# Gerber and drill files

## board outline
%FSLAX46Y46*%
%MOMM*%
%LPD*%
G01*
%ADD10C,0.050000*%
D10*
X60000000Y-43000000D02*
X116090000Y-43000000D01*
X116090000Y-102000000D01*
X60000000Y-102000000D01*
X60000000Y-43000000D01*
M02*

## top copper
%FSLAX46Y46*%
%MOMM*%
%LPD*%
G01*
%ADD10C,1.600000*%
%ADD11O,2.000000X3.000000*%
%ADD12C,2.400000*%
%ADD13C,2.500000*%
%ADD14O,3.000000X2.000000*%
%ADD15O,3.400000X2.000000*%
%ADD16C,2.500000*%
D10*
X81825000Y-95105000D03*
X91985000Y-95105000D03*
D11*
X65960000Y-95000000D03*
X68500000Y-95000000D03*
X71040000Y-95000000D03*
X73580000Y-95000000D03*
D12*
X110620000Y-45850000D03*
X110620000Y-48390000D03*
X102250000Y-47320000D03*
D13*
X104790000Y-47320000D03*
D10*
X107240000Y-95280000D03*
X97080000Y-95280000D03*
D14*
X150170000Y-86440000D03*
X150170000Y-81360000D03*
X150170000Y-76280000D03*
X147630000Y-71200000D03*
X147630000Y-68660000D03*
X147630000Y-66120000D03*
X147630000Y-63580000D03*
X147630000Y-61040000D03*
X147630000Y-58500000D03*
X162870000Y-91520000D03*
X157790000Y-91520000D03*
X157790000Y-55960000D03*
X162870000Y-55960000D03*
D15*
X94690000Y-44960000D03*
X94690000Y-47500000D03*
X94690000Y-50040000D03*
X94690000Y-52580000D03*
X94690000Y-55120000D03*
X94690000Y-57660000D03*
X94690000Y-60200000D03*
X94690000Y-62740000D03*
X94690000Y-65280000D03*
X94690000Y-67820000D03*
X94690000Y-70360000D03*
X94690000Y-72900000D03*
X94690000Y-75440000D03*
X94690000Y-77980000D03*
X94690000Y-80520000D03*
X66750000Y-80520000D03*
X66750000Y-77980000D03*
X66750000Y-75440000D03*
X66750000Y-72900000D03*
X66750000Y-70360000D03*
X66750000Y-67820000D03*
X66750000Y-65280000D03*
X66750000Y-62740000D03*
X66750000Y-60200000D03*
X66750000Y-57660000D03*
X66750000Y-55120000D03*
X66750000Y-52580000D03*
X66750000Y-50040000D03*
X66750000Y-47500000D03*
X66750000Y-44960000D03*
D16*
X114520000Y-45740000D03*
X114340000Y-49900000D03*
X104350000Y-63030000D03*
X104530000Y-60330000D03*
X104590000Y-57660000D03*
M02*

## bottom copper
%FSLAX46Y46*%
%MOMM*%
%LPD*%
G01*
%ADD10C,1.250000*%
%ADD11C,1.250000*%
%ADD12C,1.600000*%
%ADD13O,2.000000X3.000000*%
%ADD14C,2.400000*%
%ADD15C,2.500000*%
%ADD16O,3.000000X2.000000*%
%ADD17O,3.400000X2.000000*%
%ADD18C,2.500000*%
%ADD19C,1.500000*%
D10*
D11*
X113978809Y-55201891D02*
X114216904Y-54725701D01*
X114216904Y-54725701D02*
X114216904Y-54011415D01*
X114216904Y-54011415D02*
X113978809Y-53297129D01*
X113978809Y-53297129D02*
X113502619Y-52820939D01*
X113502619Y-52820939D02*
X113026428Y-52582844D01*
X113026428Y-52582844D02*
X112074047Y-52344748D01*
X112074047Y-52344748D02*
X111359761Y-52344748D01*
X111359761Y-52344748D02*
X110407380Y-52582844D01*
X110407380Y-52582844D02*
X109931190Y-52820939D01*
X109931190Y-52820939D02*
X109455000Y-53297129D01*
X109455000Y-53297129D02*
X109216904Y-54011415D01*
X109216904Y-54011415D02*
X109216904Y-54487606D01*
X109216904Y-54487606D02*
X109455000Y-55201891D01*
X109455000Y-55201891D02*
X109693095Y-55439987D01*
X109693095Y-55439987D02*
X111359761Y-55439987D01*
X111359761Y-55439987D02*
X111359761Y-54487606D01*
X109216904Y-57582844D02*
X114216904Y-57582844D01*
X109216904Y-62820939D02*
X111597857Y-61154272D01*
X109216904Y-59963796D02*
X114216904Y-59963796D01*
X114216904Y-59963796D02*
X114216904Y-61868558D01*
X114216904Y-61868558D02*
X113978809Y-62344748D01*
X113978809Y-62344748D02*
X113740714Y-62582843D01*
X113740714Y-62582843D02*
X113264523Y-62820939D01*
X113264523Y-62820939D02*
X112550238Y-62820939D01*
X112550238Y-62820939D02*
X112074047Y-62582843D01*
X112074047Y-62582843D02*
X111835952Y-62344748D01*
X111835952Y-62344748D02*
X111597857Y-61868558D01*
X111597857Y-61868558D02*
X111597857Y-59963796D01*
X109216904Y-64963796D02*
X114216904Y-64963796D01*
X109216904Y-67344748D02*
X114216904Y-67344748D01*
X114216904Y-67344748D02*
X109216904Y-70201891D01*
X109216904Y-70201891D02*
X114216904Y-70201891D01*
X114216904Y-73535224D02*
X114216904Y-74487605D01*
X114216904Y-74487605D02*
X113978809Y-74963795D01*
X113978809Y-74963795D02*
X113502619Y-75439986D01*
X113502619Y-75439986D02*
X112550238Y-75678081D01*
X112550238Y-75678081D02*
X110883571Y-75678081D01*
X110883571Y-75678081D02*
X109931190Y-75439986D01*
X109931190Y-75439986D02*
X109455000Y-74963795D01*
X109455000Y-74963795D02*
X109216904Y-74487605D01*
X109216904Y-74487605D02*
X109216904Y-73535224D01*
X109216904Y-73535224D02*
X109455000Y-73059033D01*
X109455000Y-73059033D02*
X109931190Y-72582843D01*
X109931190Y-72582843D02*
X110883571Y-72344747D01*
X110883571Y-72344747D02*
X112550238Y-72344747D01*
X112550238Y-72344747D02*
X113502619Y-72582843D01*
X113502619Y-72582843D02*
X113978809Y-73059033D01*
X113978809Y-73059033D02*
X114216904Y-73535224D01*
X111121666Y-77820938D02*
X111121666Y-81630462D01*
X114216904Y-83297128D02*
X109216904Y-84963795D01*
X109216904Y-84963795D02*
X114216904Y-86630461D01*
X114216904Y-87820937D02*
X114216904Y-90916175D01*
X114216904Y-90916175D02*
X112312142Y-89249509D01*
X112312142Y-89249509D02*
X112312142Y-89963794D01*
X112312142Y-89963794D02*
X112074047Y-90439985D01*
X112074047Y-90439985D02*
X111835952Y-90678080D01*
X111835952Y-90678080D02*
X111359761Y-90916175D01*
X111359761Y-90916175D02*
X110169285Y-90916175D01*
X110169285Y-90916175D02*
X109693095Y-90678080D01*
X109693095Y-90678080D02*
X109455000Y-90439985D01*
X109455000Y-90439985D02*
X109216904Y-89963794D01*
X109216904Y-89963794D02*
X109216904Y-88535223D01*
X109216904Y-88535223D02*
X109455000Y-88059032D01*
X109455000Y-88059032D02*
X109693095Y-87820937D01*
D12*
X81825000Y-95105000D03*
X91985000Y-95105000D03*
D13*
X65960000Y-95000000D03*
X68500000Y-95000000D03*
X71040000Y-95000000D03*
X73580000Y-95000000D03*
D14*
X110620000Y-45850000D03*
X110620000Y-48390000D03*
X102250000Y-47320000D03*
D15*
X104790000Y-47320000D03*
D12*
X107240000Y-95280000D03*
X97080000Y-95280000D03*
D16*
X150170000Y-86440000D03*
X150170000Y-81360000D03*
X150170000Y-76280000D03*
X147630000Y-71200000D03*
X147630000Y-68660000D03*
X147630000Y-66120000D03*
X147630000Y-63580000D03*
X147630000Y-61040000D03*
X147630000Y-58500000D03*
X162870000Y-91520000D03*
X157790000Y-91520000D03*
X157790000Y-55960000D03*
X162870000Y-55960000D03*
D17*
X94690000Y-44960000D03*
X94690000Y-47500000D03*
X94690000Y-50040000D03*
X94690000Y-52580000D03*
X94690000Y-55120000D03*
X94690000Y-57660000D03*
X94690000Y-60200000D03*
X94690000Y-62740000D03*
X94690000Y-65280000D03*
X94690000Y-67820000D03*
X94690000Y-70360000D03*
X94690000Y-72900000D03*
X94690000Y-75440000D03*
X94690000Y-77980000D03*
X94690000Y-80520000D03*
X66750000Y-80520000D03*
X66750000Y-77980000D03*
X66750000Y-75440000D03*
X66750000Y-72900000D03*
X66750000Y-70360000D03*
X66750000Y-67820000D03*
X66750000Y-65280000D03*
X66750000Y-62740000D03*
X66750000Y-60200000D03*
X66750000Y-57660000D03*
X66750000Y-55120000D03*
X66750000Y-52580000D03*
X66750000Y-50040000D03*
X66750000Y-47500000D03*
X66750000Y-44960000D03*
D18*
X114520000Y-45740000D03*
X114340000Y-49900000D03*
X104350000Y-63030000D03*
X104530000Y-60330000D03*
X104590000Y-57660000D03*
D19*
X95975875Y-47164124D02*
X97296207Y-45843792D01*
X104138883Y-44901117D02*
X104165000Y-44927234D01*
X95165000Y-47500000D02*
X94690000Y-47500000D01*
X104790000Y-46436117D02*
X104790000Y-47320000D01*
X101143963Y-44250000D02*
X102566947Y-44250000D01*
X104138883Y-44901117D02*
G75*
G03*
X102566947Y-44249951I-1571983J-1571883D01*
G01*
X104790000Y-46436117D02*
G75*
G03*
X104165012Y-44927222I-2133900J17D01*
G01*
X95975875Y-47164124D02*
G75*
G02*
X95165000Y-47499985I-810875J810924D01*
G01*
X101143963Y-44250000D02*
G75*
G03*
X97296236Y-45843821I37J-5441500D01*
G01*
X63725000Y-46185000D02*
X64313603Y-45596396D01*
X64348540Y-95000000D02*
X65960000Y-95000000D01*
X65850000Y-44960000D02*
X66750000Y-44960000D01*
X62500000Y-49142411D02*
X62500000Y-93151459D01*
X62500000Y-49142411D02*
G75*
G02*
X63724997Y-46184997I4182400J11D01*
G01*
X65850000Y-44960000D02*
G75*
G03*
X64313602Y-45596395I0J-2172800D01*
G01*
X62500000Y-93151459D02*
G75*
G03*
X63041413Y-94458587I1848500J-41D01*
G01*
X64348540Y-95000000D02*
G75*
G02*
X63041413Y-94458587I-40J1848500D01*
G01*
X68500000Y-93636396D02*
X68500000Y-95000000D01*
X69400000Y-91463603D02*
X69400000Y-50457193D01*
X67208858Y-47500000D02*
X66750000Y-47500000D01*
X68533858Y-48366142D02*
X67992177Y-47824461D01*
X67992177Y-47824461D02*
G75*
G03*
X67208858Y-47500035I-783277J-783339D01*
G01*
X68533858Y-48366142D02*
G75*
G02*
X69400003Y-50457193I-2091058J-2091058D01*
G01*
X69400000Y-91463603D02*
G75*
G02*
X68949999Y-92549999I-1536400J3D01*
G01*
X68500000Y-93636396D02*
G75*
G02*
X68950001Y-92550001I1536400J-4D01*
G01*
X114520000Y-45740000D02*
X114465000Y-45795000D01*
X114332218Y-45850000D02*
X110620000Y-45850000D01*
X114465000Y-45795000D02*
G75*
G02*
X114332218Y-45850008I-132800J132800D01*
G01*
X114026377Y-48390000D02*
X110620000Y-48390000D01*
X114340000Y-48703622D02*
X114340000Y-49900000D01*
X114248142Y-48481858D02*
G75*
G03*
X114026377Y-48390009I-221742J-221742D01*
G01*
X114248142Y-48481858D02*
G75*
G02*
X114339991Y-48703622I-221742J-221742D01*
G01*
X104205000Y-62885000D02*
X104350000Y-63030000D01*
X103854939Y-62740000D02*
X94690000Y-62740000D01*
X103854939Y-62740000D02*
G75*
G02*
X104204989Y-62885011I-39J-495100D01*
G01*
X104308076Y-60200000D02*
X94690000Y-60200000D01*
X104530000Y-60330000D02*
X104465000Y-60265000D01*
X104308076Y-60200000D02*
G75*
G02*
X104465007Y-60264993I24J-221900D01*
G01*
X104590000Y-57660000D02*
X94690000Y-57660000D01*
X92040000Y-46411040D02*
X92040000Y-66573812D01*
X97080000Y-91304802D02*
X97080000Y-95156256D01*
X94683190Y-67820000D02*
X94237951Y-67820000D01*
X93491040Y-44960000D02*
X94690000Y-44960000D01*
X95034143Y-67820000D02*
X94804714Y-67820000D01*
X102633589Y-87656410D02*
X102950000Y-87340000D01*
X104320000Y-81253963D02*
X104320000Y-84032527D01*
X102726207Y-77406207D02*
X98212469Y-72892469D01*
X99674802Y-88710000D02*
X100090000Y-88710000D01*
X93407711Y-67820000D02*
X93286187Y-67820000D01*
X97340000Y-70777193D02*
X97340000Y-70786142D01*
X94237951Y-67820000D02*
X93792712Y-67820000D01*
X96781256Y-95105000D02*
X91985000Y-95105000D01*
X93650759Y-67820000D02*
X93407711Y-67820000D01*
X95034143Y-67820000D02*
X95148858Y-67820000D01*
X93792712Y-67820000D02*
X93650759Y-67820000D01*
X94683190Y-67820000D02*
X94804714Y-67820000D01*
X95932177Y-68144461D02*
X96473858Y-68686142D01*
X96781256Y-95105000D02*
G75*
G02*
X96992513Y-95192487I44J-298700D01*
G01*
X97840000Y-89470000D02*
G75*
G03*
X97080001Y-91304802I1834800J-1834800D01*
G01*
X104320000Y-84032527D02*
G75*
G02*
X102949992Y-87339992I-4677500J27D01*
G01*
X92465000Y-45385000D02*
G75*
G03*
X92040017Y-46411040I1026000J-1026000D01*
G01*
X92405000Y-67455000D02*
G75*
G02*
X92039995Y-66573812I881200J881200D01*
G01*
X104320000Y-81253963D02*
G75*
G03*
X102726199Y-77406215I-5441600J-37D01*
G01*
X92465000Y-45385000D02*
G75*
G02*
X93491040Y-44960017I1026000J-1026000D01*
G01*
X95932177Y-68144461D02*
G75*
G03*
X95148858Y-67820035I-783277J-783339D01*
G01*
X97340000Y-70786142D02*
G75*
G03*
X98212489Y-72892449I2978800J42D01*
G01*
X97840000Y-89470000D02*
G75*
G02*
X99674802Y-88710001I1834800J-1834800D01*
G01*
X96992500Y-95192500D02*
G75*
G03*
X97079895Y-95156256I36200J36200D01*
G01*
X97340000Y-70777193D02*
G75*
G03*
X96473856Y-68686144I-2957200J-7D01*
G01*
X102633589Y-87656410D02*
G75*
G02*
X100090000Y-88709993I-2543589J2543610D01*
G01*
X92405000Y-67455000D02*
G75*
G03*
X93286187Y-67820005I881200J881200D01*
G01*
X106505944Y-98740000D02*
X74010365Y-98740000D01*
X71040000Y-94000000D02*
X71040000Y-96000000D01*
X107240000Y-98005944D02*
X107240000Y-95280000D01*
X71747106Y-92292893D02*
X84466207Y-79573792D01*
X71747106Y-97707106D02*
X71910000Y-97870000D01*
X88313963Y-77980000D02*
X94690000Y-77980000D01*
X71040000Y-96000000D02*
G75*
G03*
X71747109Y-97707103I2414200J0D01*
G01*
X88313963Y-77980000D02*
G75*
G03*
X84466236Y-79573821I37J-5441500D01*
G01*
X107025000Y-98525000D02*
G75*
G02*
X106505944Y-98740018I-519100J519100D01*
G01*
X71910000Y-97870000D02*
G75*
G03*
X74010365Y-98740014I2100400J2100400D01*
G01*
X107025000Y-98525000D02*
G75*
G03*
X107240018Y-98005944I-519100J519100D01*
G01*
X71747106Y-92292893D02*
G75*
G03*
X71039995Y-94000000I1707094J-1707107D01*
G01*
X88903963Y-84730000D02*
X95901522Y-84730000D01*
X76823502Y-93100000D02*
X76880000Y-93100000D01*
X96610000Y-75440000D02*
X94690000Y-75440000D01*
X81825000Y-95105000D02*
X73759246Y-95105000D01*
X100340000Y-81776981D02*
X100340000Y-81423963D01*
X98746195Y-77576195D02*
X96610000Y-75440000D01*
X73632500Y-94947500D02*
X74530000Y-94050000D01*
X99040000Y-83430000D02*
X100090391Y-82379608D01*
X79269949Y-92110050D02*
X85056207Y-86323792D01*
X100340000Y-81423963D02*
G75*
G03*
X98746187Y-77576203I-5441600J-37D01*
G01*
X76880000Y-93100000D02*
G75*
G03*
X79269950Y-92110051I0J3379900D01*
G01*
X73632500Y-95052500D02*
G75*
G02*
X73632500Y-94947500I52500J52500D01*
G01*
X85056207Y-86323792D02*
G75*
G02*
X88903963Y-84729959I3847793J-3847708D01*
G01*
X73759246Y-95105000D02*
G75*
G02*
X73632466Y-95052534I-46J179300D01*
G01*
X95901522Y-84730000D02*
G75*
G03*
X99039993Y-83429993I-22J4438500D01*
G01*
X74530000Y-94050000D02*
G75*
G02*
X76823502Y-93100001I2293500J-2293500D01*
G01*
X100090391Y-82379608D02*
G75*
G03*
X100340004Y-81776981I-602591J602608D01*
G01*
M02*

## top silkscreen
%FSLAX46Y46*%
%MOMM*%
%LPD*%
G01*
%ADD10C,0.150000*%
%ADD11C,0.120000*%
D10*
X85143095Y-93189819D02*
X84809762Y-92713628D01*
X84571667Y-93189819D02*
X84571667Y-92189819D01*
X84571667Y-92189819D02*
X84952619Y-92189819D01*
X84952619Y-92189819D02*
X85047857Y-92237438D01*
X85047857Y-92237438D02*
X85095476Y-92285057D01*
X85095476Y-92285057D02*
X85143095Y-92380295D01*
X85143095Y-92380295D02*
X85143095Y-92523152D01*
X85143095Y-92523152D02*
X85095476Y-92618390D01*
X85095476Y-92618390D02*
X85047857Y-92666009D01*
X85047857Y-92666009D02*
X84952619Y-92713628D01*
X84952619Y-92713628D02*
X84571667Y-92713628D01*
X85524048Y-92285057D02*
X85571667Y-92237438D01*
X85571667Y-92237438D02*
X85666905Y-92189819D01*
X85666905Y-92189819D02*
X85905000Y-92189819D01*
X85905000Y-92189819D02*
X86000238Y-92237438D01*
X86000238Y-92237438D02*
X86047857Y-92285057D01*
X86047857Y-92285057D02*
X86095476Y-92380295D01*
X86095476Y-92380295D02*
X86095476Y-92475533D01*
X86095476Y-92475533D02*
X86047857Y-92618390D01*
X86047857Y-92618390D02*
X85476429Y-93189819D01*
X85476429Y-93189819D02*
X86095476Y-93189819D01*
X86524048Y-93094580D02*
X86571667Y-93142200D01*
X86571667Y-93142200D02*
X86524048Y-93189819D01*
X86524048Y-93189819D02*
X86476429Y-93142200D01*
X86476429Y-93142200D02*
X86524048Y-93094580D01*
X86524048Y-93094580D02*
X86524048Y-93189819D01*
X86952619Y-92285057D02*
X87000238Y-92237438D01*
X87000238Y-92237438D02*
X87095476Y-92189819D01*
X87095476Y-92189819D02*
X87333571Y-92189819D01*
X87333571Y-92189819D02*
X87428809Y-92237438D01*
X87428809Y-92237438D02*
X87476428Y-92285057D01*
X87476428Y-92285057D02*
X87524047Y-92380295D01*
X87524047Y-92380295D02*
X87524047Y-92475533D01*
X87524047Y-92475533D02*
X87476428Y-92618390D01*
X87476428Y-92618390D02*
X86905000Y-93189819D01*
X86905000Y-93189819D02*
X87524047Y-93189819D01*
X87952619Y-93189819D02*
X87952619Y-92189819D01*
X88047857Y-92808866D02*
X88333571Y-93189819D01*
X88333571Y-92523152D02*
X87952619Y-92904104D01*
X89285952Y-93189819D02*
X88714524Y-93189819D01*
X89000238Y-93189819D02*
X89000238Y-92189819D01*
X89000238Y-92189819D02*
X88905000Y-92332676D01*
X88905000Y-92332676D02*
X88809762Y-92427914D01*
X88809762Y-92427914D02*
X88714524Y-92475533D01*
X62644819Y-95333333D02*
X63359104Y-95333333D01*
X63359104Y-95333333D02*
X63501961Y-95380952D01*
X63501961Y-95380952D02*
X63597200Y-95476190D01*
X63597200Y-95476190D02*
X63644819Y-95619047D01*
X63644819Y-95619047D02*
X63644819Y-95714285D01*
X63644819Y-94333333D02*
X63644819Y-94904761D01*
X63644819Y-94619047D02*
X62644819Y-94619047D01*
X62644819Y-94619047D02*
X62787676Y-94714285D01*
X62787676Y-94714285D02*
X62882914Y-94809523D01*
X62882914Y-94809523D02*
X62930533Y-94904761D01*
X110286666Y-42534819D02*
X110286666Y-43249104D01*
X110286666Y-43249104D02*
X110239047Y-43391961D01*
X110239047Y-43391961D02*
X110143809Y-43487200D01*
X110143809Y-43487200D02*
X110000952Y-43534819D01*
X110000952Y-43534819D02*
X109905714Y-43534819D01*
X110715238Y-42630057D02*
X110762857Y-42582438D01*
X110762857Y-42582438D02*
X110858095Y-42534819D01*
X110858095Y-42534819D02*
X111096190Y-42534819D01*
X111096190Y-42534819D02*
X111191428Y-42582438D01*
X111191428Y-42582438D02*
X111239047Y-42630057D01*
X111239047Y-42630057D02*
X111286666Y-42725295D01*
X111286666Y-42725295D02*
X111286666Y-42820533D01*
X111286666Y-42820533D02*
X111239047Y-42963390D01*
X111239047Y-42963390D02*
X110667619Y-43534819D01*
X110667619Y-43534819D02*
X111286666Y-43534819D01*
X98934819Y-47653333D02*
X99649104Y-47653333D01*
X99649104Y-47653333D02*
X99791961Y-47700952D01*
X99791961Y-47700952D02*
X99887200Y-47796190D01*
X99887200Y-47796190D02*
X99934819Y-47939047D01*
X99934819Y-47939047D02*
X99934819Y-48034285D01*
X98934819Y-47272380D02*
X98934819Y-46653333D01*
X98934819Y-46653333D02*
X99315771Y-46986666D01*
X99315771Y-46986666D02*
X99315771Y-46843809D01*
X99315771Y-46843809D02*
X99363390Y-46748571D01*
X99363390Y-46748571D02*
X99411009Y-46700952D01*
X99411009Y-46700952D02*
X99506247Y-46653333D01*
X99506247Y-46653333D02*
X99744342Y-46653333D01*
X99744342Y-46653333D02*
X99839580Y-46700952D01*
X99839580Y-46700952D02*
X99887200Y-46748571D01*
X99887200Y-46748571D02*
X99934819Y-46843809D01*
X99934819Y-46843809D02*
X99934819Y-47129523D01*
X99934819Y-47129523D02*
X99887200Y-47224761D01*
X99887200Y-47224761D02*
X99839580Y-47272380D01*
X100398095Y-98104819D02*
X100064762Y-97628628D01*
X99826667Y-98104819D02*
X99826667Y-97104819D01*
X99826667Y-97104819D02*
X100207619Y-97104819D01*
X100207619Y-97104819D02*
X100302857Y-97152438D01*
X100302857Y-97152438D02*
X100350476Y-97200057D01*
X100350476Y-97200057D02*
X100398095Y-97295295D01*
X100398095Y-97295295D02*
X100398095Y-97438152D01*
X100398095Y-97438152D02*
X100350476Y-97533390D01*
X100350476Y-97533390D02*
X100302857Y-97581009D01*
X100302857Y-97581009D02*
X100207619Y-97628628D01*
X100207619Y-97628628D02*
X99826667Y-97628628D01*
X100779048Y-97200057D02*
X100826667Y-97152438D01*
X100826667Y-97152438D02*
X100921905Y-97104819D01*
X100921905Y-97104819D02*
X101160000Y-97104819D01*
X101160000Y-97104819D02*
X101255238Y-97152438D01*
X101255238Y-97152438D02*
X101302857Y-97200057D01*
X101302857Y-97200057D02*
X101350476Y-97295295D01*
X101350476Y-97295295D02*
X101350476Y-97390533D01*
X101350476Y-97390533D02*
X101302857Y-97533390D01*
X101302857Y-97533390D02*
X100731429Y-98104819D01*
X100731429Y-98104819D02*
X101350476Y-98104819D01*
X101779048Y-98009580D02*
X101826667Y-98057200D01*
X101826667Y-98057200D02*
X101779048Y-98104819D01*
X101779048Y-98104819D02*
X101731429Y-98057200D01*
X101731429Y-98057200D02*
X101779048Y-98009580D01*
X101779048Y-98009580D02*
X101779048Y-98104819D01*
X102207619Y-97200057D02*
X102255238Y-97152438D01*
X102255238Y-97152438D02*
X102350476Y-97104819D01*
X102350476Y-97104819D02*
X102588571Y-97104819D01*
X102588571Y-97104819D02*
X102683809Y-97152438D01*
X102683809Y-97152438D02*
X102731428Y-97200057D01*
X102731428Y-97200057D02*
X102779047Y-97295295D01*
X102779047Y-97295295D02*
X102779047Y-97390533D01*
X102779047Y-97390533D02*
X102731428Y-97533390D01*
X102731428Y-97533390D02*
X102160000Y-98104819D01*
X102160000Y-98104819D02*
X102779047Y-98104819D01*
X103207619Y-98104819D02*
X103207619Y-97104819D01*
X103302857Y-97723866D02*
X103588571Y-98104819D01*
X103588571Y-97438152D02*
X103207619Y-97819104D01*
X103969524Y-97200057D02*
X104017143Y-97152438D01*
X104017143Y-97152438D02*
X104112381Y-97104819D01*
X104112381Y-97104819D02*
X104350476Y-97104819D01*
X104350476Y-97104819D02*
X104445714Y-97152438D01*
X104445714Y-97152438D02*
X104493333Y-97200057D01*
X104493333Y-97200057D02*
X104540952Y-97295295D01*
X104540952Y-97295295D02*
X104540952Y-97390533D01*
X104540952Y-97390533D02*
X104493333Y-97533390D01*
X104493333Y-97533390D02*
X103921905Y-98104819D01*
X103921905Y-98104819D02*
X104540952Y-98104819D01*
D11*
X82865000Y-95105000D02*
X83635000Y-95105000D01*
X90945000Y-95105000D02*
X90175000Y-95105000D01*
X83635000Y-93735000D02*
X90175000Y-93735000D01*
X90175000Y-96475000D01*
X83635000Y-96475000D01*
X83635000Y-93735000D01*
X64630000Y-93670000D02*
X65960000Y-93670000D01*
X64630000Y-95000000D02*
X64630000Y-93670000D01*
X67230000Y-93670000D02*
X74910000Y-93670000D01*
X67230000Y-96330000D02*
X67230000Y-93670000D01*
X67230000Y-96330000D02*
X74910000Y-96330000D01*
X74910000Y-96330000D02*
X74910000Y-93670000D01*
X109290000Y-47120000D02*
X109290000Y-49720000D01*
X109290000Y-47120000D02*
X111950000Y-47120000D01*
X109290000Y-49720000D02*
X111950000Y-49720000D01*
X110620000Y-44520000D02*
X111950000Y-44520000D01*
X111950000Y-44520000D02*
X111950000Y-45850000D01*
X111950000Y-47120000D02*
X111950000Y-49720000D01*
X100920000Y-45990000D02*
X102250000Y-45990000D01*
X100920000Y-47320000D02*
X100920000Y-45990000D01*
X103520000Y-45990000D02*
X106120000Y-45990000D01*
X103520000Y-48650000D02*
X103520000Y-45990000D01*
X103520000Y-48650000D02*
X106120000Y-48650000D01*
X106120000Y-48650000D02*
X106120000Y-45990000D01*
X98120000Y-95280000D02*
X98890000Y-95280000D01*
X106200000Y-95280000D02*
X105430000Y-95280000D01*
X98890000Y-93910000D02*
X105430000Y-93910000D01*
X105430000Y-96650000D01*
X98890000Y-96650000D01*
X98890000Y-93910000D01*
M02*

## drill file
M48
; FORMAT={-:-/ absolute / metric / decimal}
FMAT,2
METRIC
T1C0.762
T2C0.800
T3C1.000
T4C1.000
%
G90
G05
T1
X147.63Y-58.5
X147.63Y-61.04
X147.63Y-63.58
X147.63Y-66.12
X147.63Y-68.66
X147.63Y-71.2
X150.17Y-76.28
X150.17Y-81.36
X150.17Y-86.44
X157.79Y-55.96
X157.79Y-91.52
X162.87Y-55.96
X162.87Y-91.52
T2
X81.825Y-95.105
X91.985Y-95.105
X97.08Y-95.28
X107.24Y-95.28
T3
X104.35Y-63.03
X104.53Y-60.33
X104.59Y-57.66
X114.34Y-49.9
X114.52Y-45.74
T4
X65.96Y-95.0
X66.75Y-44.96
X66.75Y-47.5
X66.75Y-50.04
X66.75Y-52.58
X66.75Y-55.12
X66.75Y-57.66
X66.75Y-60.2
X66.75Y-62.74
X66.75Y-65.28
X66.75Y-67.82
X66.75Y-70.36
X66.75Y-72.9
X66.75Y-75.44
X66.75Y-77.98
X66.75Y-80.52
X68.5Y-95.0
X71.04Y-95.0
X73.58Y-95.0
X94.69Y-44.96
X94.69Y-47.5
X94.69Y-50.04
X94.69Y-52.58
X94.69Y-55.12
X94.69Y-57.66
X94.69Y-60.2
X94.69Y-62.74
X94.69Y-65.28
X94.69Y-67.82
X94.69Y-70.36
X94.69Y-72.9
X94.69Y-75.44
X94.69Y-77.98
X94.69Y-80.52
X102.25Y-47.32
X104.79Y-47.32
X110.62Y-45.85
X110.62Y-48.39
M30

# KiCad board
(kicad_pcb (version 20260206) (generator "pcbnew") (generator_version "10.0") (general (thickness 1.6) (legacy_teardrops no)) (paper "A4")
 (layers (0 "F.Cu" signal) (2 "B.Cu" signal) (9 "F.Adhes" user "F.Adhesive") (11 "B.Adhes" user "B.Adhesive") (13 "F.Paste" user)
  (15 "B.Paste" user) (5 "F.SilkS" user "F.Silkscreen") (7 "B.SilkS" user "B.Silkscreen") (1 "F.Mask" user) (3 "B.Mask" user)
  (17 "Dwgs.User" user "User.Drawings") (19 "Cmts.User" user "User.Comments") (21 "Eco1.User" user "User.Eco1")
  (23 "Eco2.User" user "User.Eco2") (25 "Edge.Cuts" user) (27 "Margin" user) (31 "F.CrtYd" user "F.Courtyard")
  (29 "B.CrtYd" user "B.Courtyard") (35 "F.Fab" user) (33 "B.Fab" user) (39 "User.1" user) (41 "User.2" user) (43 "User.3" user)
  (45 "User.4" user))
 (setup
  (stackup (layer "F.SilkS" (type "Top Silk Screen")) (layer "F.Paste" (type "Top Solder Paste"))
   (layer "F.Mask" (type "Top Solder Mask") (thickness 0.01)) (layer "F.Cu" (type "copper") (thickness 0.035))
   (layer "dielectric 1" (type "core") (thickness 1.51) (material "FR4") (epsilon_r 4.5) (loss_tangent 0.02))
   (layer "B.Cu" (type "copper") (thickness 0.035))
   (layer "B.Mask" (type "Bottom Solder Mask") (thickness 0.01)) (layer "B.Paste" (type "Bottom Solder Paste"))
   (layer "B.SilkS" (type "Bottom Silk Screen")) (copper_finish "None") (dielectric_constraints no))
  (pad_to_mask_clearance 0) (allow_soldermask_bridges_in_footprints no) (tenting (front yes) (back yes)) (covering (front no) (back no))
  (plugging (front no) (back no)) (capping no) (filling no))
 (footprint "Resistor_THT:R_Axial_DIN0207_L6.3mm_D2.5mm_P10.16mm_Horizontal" (layer "F.Cu") (at 81.825 95.105)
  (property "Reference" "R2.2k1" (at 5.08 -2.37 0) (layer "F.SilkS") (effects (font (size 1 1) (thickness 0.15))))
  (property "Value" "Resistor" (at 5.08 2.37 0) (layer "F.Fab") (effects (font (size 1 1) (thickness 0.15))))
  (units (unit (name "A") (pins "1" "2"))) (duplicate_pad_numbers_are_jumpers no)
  (fp_line (start 1.04 0) (end 1.81 0) (stroke (width 0.12) (type solid)) (layer "F.SilkS"))
  (fp_line (start 9.12 0) (end 8.35 0) (stroke (width 0.12) (type solid)) (layer "F.SilkS"))
  (fp_rect (start 1.81 -1.37) (end 8.35 1.37) (stroke (width 0.12) (type solid)) (fill no) (layer "F.SilkS"))
  (pad "1" thru_hole circle (at 0 0) (size 1.6 1.6) (drill 0.8) (layers "*.Cu" "*.Mask") (remove_unused_layers no)
   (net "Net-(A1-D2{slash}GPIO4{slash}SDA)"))
  (pad "2" thru_hole circle (at 10.16 0) (size 1.6 1.6) (drill 0.8) (layers "*.Cu" "*.Mask") (remove_unused_layers no) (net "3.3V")))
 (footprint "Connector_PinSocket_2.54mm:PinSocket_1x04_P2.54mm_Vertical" (layer "F.Cu") (at 65.96 95 90)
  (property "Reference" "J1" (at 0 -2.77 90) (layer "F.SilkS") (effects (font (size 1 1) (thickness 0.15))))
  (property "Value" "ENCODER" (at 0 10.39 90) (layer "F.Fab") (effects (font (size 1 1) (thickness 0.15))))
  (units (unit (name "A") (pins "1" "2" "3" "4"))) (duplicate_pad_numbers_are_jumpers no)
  (fp_line (start 1.33 -1.33) (end 1.33 0) (stroke (width 0.12) (type solid)) (layer "F.SilkS"))
  (fp_line (start 0 -1.33) (end 1.33 -1.33) (stroke (width 0.12) (type solid)) (layer "F.SilkS"))
  (fp_line (start 1.33 1.27) (end 1.33 8.95) (stroke (width 0.12) (type solid)) (layer "F.SilkS"))
  (fp_line (start -1.33 1.27) (end 1.33 1.27) (stroke (width 0.12) (type solid)) (layer "F.SilkS"))
  (fp_line (start -1.33 1.27) (end -1.33 8.95) (stroke (width 0.12) (type solid)) (layer "F.SilkS"))
  (fp_line (start -1.33 8.95) (end 1.33 8.95) (stroke (width 0.12) (type solid)) (layer "F.SilkS"))
  (pad "1" thru_hole oval (at 0 0 90) (size 3 2) (drill 1) (layers "*.Cu" "*.Mask") (remove_unused_layers no) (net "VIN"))
  (pad "2" thru_hole oval (at 0 2.54 90) (size 3 2) (drill 1) (layers "*.Cu" "*.Mask") (remove_unused_layers no) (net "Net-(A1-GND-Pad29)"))
  (pad "3" thru_hole oval (at 0 5.08 90) (size 3 2) (drill 1) (layers "*.Cu" "*.Mask") (remove_unused_layers no)
   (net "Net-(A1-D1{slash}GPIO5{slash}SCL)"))
  (pad "4" thru_hole oval (at 0 7.62 90) (size 3 2) (drill 1) (layers "*.Cu" "*.Mask") (remove_unused_layers no)
   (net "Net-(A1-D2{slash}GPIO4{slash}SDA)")))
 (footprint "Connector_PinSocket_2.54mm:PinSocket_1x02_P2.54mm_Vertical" (layer "F.Cu") (at 110.62 45.85)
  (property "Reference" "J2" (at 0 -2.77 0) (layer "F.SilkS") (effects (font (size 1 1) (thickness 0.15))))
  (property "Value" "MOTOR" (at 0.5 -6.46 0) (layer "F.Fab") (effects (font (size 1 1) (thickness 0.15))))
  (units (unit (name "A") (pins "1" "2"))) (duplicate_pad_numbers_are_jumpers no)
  (fp_line (start -1.33 1.27) (end -1.33 3.87) (stroke (width 0.12) (type solid)) (layer "F.SilkS"))
  (fp_line (start -1.33 1.27) (end 1.33 1.27) (stroke (width 0.12) (type solid)) (layer "F.SilkS"))
  (fp_line (start -1.33 3.87) (end 1.33 3.87) (stroke (width 0.12) (type solid)) (layer "F.SilkS"))
  (fp_line (start 0 -1.33) (end 1.33 -1.33) (stroke (width 0.12) (type solid)) (layer "F.SilkS"))
  (fp_line (start 1.33 -1.33) (end 1.33 0) (stroke (width 0.12) (type solid)) (layer "F.SilkS"))
  (fp_line (start 1.33 1.27) (end 1.33 3.87) (stroke (width 0.12) (type solid)) (layer "F.SilkS"))
  (pad "1" thru_hole circle (at 0 0) (size 2.4 2.4) (drill 1) (layers "*.Cu" "*.Mask") (remove_unused_layers no) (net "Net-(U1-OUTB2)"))
  (pad "2" thru_hole circle (at 0 2.54) (size 2.4 2.4) (drill 1) (layers "*.Cu" "*.Mask") (remove_unused_layers no) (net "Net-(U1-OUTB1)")))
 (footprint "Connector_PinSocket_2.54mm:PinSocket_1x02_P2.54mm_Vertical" (layer "F.Cu") (at 102.25 47.32 90)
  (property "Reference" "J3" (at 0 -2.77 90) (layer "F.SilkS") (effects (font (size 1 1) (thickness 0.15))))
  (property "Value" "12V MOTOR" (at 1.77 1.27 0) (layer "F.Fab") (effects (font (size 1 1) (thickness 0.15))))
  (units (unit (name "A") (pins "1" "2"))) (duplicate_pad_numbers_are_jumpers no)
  (fp_line (start 1.33 -1.33) (end 1.33 0) (stroke (width 0.12) (type solid)) (layer "F.SilkS"))
  (fp_line (start 0 -1.33) (end 1.33 -1.33) (stroke (width 0.12) (type solid)) (layer "F.SilkS"))
  (fp_line (start 1.33 1.27) (end 1.33 3.87) (stroke (width 0.12) (type solid)) (layer "F.SilkS"))
  (fp_line (start -1.33 1.27) (end 1.33 1.27) (stroke (width 0.12) (type solid)) (layer "F.SilkS"))
  (fp_line (start -1.33 1.27) (end -1.33 3.87) (stroke (width 0.12) (type solid)) (layer "F.SilkS"))
  (fp_line (start -1.33 3.87) (end 1.33 3.87) (stroke (width 0.12) (type solid)) (layer "F.SilkS"))
  (pad "1" thru_hole circle (at 0 0 90) (size 2.4 2.4) (drill 1) (layers "*.Cu" "*.Mask") (remove_unused_layers no) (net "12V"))
  (pad "2" thru_hole circle (at 0 2.54 90) (size 2.5 2.5) (drill 1) (layers "*.Cu" "*.Mask") (remove_unused_layers no) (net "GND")))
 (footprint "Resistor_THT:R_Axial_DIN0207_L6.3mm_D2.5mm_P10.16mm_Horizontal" (layer "F.Cu") (at 107.24 95.28 180)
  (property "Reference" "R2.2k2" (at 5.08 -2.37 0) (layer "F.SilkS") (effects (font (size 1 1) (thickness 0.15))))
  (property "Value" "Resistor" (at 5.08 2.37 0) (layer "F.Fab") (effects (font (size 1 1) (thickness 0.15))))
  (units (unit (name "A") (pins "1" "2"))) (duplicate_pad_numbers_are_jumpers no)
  (fp_line (start 9.12 0) (end 8.35 0) (stroke (width 0.12) (type solid)) (layer "F.SilkS"))
  (fp_line (start 1.04 0) (end 1.81 0) (stroke (width 0.12) (type solid)) (layer "F.SilkS"))
  (fp_rect (start 1.81 -1.37) (end 8.35 1.37) (stroke (width 0.12) (type solid)) (fill no) (layer "F.SilkS"))
  (pad "1" thru_hole circle (at 0 0 180) (size 1.6 1.6) (drill 0.8) (layers "*.Cu" "*.Mask") (remove_unused_layers no)
   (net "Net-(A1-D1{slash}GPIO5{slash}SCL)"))
  (pad "2" thru_hole circle (at 10.16 0 180) (size 1.6 1.6) (drill 0.8) (layers "*.Cu" "*.Mask") (remove_unused_layers no) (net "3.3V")))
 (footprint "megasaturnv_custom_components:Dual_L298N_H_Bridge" (layer "B.Cu") (at 145.09 94.06 90)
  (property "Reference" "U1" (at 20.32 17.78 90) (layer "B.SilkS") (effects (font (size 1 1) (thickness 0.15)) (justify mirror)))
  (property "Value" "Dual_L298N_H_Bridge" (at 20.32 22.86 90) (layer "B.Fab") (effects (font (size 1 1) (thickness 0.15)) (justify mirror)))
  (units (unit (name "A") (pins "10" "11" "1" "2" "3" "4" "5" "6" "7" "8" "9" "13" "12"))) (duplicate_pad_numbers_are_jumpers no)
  (pad "1" thru_hole oval (at 7.62 5.08 90) (size 2 3) (drill 0.762) (layers "*.Cu" "*.Mask") (remove_unused_layers no)
   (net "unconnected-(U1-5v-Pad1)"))
  (pad "2" thru_hole oval (at 12.7 5.08 90) (size 2 3) (drill 0.762) (layers "*.Cu" "*.Mask") (remove_unused_layers no) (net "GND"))
  (pad "3" thru_hole oval (at 17.78 5.08 90) (size 2 3) (drill 0.762) (layers "*.Cu" "*.Mask") (remove_unused_layers no) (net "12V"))
  (pad "4" thru_hole oval (at 22.86 2.54 90) (size 2 3) (drill 0.762) (layers "*.Cu" "*.Mask") (remove_unused_layers no)
   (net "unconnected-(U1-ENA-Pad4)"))
  (pad "5" thru_hole oval (at 25.4 2.54 90) (size 2 3) (drill 0.762) (layers "*.Cu" "*.Mask") (remove_unused_layers no)
   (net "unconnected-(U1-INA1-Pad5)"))
  (pad "6" thru_hole oval (at 27.94 2.54 90) (size 2 3) (drill 0.762) (layers "*.Cu" "*.Mask") (remove_unused_layers no)
   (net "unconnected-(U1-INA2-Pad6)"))
  (pad "7" thru_hole oval (at 30.48 2.54 90) (size 2 3) (drill 0.762) (layers "*.Cu" "*.Mask") (remove_unused_layers no)
   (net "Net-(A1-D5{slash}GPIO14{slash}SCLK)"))
  (pad "8" thru_hole oval (at 33.02 2.54 90) (size 2 3) (drill 0.762) (layers "*.Cu" "*.Mask") (remove_unused_layers no)
   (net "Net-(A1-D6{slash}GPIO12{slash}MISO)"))
  (pad "9" thru_hole oval (at 35.56 2.54 90) (size 2 3) (drill 0.762) (layers "*.Cu" "*.Mask") (remove_unused_layers no)
   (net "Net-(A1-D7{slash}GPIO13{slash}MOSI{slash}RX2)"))
  (pad "10" thru_hole oval (at 2.54 17.78 90) (size 2 3) (drill 0.762) (layers "*.Cu" "*.Mask") (remove_unused_layers no)
   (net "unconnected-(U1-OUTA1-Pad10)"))
  (pad "11" thru_hole oval (at 2.54 12.7 90) (size 2 3) (drill 0.762) (layers "*.Cu" "*.Mask") (remove_unused_layers no)
   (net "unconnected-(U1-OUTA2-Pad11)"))
  (pad "12" thru_hole oval (at 38.1 12.7 90) (size 2 3) (drill 0.762) (layers "*.Cu" "*.Mask") (remove_unused_layers no)
   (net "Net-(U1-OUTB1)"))
  (pad "13" thru_hole oval (at 38.1 17.78 90) (size 2 3) (drill 0.762) (layers "*.Cu" "*.Mask") (remove_unused_layers no)
   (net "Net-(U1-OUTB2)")))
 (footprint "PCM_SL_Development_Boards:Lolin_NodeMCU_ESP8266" (layer "B.Cu") (at 80.72 62.74 180)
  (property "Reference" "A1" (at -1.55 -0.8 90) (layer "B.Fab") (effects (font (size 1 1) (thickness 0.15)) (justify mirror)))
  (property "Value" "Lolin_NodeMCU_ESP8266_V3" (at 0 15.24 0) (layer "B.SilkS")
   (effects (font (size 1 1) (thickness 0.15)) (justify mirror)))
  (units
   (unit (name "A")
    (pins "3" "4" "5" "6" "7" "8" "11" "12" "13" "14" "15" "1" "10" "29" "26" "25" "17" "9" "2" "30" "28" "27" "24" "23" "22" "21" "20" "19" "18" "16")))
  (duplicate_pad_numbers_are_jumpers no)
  (pad "1" thru_hole oval (at -13.97 17.78 270) (size 2 3.4) (drill 1) (layers "*.Cu" "*.Mask") (remove_unused_layers no)
   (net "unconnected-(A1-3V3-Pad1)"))
  (pad "2" thru_hole oval (at -13.97 15.24 270) (size 2 3.4) (drill 1) (layers "*.Cu" "*.Mask") (remove_unused_layers no) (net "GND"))
  (pad "3" thru_hole oval (at -13.97 12.7 270) (size 2 3.4) (drill 1) (layers "*.Cu" "*.Mask") (remove_unused_layers no)
   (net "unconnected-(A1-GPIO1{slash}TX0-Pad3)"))
  (pad "4" thru_hole oval (at -13.97 10.16 270) (size 2 3.4) (drill 1) (layers "*.Cu" "*.Mask") (remove_unused_layers no)
   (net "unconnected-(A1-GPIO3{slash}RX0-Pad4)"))
  (pad "5" thru_hole oval (at -13.97 7.62 270) (size 2 3.4) (drill 1) (layers "*.Cu" "*.Mask") (remove_unused_layers no)
   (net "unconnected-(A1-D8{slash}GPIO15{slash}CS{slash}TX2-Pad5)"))
  (pad "6" thru_hole oval (at -13.97 5.08 270) (size 2 3.4) (drill 1) (layers "*.Cu" "*.Mask") (remove_unused_layers no)
   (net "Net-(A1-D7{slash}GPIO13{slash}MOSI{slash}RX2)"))
  (pad "7" thru_hole oval (at -13.97 2.54 270) (size 2 3.4) (drill 1) (layers "*.Cu" "*.Mask") (remove_unused_layers no)
   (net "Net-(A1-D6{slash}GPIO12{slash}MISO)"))
  (pad "8" thru_hole oval (at -13.97 0 270) (size 2 3.4) (drill 1) (layers "*.Cu" "*.Mask") (remove_unused_layers no)
   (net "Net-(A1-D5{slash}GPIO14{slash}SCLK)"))
  (pad "9" thru_hole oval (at -13.97 -2.54 270) (size 2 3.4) (drill 1) (layers "*.Cu" "*.Mask") (remove_unused_layers no)
   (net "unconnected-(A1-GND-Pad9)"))
  (pad "10" thru_hole oval (at -13.97 -5.08 270) (size 2 3.4) (drill 1) (layers "*.Cu" "*.Mask") (remove_unused_layers no) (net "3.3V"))
  (pad "11" thru_hole oval (at -13.97 -7.62 270) (size 2 3.4) (drill 1) (layers "*.Cu" "*.Mask") (remove_unused_layers no)
   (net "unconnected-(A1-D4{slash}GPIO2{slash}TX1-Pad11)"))
  (pad "12" thru_hole oval (at -13.97 -10.16 270) (size 2 3.4) (drill 1) (layers "*.Cu" "*.Mask") (remove_unused_layers no)
   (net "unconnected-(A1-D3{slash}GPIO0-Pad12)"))
  (pad "13" thru_hole oval (at -13.97 -12.7 270) (size 2 3.4) (drill 1) (layers "*.Cu" "*.Mask") (remove_unused_layers no)
   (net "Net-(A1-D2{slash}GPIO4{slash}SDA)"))
  (pad "14" thru_hole oval (at -13.97 -15.24 270) (size 2 3.4) (drill 1) (layers "*.Cu" "*.Mask") (remove_unused_layers no)
   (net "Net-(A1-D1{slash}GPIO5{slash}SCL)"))
  (pad "15" thru_hole oval (at -13.97 -17.78 270) (size 2 3.4) (drill 1) (layers "*.Cu" "*.Mask") (remove_unused_layers no)
   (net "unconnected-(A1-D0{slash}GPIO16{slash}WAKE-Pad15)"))
  (pad "16" thru_hole oval (at 13.97 -17.78 270) (size 2 3.4) (drill 1) (layers "*.Cu" "*.Mask") (remove_unused_layers no)
   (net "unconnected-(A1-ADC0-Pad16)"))
  (pad "17" thru_hole oval (at 13.97 -15.24 270) (size 2 3.4) (drill 1) (layers "*.Cu" "*.Mask") (remove_unused_layers no)
   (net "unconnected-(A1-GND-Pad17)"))
  (pad "18" thru_hole oval (at 13.97 -12.7 270) (size 2 3.4) (drill 1) (layers "*.Cu" "*.Mask") (remove_unused_layers no)
   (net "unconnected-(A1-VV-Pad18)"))
  (pad "19" thru_hole oval (at 13.97 -10.16 270) (size 2 3.4) (drill 1) (layers "*.Cu" "*.Mask") (remove_unused_layers no)
   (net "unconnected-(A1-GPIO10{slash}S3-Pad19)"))
  (pad "20" thru_hole oval (at 13.97 -7.62 270) (size 2 3.4) (drill 1) (layers "*.Cu" "*.Mask") (remove_unused_layers no)
   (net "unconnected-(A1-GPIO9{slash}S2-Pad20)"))
  (pad "21" thru_hole oval (at 13.97 -5.08 270) (size 2 3.4) (drill 1) (layers "*.Cu" "*.Mask") (remove_unused_layers no)
   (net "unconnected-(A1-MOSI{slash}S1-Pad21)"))
  (pad "22" thru_hole oval (at 13.97 -2.54 270) (size 2 3.4) (drill 1) (layers "*.Cu" "*.Mask") (remove_unused_layers no)
   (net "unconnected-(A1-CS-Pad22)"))
  (pad "23" thru_hole oval (at 13.97 0 270) (size 2 3.4) (drill 1) (layers "*.Cu" "*.Mask") (remove_unused_layers no)
   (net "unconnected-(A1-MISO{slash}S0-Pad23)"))
  (pad "24" thru_hole oval (at 13.97 2.54 270) (size 2 3.4) (drill 1) (layers "*.Cu" "*.Mask") (remove_unused_layers no)
   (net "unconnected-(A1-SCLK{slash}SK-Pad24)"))
  (pad "25" thru_hole oval (at 13.97 5.08 270) (size 2 3.4) (drill 1) (layers "*.Cu" "*.Mask") (remove_unused_layers no)
   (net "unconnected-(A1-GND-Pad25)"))
  (pad "26" thru_hole oval (at 13.97 7.62 270) (size 2 3.4) (drill 1) (layers "*.Cu" "*.Mask") (remove_unused_layers no)
   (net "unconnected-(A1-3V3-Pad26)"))
  (pad "27" thru_hole oval (at 13.97 10.16 270) (size 2 3.4) (drill 1) (layers "*.Cu" "*.Mask") (remove_unused_layers no)
   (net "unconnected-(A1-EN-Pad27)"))
  (pad "28" thru_hole oval (at 13.97 12.7 270) (size 2 3.4) (drill 1) (layers "*.Cu" "*.Mask") (remove_unused_layers no)
   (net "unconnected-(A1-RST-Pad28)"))
  (pad "29" thru_hole oval (at 13.97 15.24 270) (size 2 3.4) (drill 1) (layers "*.Cu" "*.Mask") (remove_unused_layers no)
   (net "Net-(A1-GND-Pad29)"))
  (pad "30" thru_hole oval (at 13.97 17.78 270) (size 2 3.4) (drill 1) (layers "*.Cu" "*.Mask") (remove_unused_layers no) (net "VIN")))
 (gr_rect (start 60 43) (end 116.09 102) (stroke (width 0.05) (type default)) (fill no) (layer "Edge.Cuts"))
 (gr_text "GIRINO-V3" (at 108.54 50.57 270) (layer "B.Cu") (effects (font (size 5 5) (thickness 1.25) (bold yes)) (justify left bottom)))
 (segment (start 95.975875 47.164124) (end 97.296207 45.843792) (width 1.5) (layer "B.Cu") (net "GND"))
 (segment (start 104.138883 44.901117) (end 104.165 44.927234) (width 1.5) (layer "B.Cu") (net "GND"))
 (segment (start 95.165 47.5) (end 94.69 47.5) (width 1.5) (layer "B.Cu") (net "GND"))
 (segment (start 104.79 46.436117) (end 104.79 47.32) (width 1.5) (layer "B.Cu") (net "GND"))
 (segment (start 101.143963 44.25) (end 102.566947 44.25) (width 1.5) (layer "B.Cu") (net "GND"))
 (arc (start 104.138883 44.901117) (mid 103.417672 44.419219) (end 102.566947 44.25) (width 1.5) (layer "B.Cu") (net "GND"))
 (arc (start 104.79 46.436117) (mid 104.627567 45.619515) (end 104.165 44.927234) (width 1.5) (layer "B.Cu") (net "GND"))
 (arc (start 95.975875 47.164124) (mid 95.603842 47.412708) (end 95.165 47.5) (width 1.5) (layer "B.Cu") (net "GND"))
 (arc (start 101.143963 44.25) (mid 99.061572 44.664213) (end 97.296207 45.843792) (width 1.5) (layer "B.Cu") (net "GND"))
 (segment (start 63.725 46.185) (end 64.313603 45.596396) (width 1.5) (layer "B.Cu") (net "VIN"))
 (segment (start 64.34854 95) (end 65.96 95) (width 1.5) (layer "B.Cu") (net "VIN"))
 (segment (start 65.85 44.96) (end 66.75 44.96) (width 1.5) (layer "B.Cu") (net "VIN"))
 (segment (start 62.5 49.142411) (end 62.5 93.151459) (width 1.5) (layer "B.Cu") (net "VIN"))
 (arc (start 62.5 49.142411) (mid 62.818367 47.541871) (end 63.725 46.185) (width 1.5) (layer "B.Cu") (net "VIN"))
 (arc (start 65.85 44.96) (mid 65.018508 45.125393) (end 64.313603 45.596396) (width 1.5) (layer "B.Cu") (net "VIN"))
 (arc (start 62.5 93.151459) (mid 62.640711 93.858865) (end 63.041425 94.458575) (width 1.5) (layer "B.Cu") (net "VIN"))
 (arc (start 64.34854 95) (mid 63.641134 94.859288) (end 63.041425 94.458575) (width 1.5) (layer "B.Cu") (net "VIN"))
 (segment (start 68.5 93.636396) (end 68.5 95) (width 1.5) (layer "B.Cu") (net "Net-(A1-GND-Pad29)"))
 (segment (start 69.4 91.463603) (end 69.4 50.457193) (width 1.5) (layer "B.Cu") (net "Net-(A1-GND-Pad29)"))
 (segment (start 67.208858 47.5) (end 66.75 47.5) (width 1.5) (layer "B.Cu") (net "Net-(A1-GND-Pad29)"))
 (segment (start 68.533858 48.366142) (end 67.992177 47.824461) (width 1.5) (layer "B.Cu") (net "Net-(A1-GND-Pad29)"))
 (arc (start 67.992177 47.824461) (mid 67.632787 47.584324) (end 67.208858 47.5) (width 1.5) (layer "B.Cu") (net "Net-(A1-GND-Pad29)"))
 (arc (start 68.533858 48.366142) (mid 69.174897 49.325524) (end 69.4 50.457193) (width 1.5) (layer "B.Cu") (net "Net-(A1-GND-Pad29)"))
 (arc (start 69.4 91.463603) (mid 69.283048 92.051556) (end 68.95 92.55) (width 1.5) (layer "B.Cu") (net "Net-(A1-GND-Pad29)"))
 (arc (start 68.5 93.636396) (mid 68.616951 93.048442) (end 68.95 92.55) (width 1.5) (layer "B.Cu") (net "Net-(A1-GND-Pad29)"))
 (via (at 114.52 45.74) (size 2.5) (drill 1) (layers "F.Cu" "B.Cu") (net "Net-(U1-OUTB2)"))
 (segment (start 114.52 45.74) (end 114.465 45.795) (width 1.5) (layer "B.Cu") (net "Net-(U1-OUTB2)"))
 (segment (start 114.332218 45.85) (end 110.62 45.85) (width 1.5) (layer "B.Cu") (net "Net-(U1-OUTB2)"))
 (arc (start 114.465 45.795) (mid 114.404079 45.835705) (end 114.332218 45.85) (width 1.5) (layer "B.Cu") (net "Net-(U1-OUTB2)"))
 (via (at 114.34 49.9) (size 2.5) (drill 1) (layers "F.Cu" "B.Cu") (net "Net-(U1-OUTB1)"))
 (segment (start 114.026377 48.39) (end 110.62 48.39) (width 1.5) (layer "B.Cu") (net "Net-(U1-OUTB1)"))
 (segment (start 114.34 48.703622) (end 114.34 49.9) (width 1.5) (layer "B.Cu") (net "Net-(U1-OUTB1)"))
 (arc (start 114.248142 48.481858) (mid 114.146395 48.413873) (end 114.026377 48.39) (width 1.5) (layer "B.Cu") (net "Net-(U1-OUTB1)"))
 (arc (start 114.248142 48.481858) (mid 114.316126 48.583604) (end 114.34 48.703622) (width 1.5) (layer "B.Cu") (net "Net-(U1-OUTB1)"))
 (via (at 104.35 63.03) (size 2.5) (drill 1) (layers "F.Cu" "B.Cu") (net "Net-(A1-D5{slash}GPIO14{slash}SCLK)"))
 (segment (start 104.205 62.885) (end 104.35 63.03) (width 1.5) (layer "B.Cu") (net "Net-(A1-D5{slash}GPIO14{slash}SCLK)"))
 (segment (start 103.854939 62.74) (end 94.69 62.74) (width 1.5) (layer "B.Cu") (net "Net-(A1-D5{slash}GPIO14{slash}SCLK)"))
 (arc (start 103.854939 62.74) (mid 104.04439 62.777684) (end 104.205 62.885) (width 1.5) (layer "B.Cu")
  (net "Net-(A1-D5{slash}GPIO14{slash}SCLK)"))
 (via (at 104.53 60.33) (size 2.5) (drill 1) (layers "F.Cu" "B.Cu") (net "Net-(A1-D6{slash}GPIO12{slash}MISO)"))
 (segment (start 104.308076 60.2) (end 94.69 60.2) (width 1.5) (layer "B.Cu") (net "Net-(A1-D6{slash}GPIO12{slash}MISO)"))
 (segment (start 104.53 60.33) (end 104.465 60.265) (width 1.5) (layer "B.Cu") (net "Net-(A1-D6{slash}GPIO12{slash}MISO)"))
 (arc (start 104.308076 60.2) (mid 104.393002 60.216892) (end 104.465 60.265) (width 1.5) (layer "B.Cu")
  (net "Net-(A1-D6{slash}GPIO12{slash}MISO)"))
 (via (at 104.59 57.66) (size 2.5) (drill 1) (layers "F.Cu" "B.Cu") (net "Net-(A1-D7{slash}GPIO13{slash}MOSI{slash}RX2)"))
 (segment (start 104.59 57.66) (end 94.69 57.66) (width 1.5) (layer "B.Cu") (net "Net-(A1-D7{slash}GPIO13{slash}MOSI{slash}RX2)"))
 (segment (start 92.04 46.41104) (end 92.04 66.573812) (width 1.5) (layer "B.Cu") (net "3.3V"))
 (segment (start 97.08 91.304802) (end 97.08 95.156256) (width 1.5) (layer "B.Cu") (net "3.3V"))
 (segment (start 94.68319 67.82) (end 94.237951 67.82) (width 1.5) (layer "B.Cu") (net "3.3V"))
 (segment (start 93.49104 44.96) (end 94.69 44.96) (width 1.5) (layer "B.Cu") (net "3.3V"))
 (segment (start 95.034143 67.82) (end 94.804714 67.82) (width 1.5) (layer "B.Cu") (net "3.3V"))
 (segment (start 102.633589 87.65641) (end 102.95 87.34) (width 1.5) (layer "B.Cu") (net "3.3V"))
 (segment (start 104.32 81.253963) (end 104.32 84.032527) (width 1.5) (layer "B.Cu") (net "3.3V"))
 (segment (start 102.726207 77.406207) (end 98.212469 72.892469) (width 1.5) (layer "B.Cu") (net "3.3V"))
 (segment (start 99.674802 88.71) (end 100.09 88.71) (width 1.5) (layer "B.Cu") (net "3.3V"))
 (segment (start 93.407711 67.82) (end 93.286187 67.82) (width 1.5) (layer "B.Cu") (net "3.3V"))
 (segment (start 97.34 70.777193) (end 97.34 70.786142) (width 1.5) (layer "B.Cu") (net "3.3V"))
 (segment (start 94.237951 67.82) (end 93.792712 67.82) (width 1.5) (layer "B.Cu") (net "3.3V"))
 (segment (start 96.781256 95.105) (end 91.985 95.105) (width 1.5) (layer "B.Cu") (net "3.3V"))
 (segment (start 93.650759 67.82) (end 93.407711 67.82) (width 1.5) (layer "B.Cu") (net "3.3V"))
 (segment (start 95.034143 67.82) (end 95.148858 67.82) (width 1.5) (layer "B.Cu") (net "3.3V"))
 (segment (start 93.792712 67.82) (end 93.650759 67.82) (width 1.5) (layer "B.Cu") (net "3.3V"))
 (segment (start 94.68319 67.82) (end 94.804714 67.82) (width 1.5) (layer "B.Cu") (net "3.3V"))
 (segment (start 95.932177 68.144461) (end 96.473858 68.686142) (width 1.5) (layer "B.Cu") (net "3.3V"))
 (arc (start 96.781256 95.105) (mid 96.89558 95.12774) (end 96.9925 95.1925) (width 1.5) (layer "B.Cu") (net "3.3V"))
 (arc (start 97.84 89.47) (mid 97.277517 90.311814) (end 97.08 91.304802) (width 1.5) (layer "B.Cu") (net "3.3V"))
 (arc (start 104.32 84.032527) (mid 103.963948 85.822518) (end 102.95 87.34) (width 1.5) (layer "B.Cu") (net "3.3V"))
 (arc (start 92.465 45.385) (mid 92.150453 45.855751) (end 92.04 46.41104) (width 1.5) (layer "B.Cu") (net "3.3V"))
 (arc (start 92.405 67.455) (mid 92.13486 67.050707) (end 92.04 66.573812) (width 1.5) (layer "B.Cu") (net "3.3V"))
 (arc (start 104.32 81.253963) (mid 103.905786 79.171572) (end 102.726207 77.406207) (width 1.5) (layer "B.Cu") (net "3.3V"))
 (arc (start 92.465 45.385) (mid 92.935751 45.070453) (end 93.49104 44.96) (width 1.5) (layer "B.Cu") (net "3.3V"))
 (arc (start 95.932177 68.144461) (mid 95.572787 67.904324) (end 95.148858 67.82) (width 1.5) (layer "B.Cu") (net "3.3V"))
 (arc (start 97.34 70.786142) (mid 97.566747 71.926078) (end 98.212469 72.892469) (width 1.5) (layer "B.Cu") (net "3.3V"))
 (arc (start 97.84 89.47) (mid 98.681814 88.907517) (end 99.674802 88.71) (width 1.5) (layer "B.Cu") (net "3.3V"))
 (arc (start 96.9925 95.1925) (mid 97.048358 95.20361) (end 97.08 95.156256) (width 1.5) (layer "B.Cu") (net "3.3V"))
 (arc (start 97.34 70.777193) (mid 97.114897 69.645524) (end 96.473858 68.686142) (width 1.5) (layer "B.Cu") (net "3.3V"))
 (arc (start 102.633589 87.65641) (mid 101.46658 88.43618) (end 100.09 88.71) (width 1.5) (layer "B.Cu") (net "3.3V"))
 (arc (start 92.405 67.455) (mid 92.809292 67.725139) (end 93.286187 67.82) (width 1.5) (layer "B.Cu") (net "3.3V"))
 (segment (start 106.505944 98.74) (end 74.010365 98.74) (width 1.5) (layer "B.Cu") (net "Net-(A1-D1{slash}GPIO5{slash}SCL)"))
 (segment (start 71.04 94) (end 71.04 96) (width 1.5) (layer "B.Cu") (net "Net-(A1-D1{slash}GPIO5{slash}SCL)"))
 (segment (start 107.24 98.005944) (end 107.24 95.28) (width 1.5) (layer "B.Cu") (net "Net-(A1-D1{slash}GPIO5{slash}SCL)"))
 (segment (start 71.747106 92.292893) (end 84.466207 79.573792) (width 1.5) (layer "B.Cu") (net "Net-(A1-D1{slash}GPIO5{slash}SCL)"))
 (segment (start 71.747106 97.707106) (end 71.91 97.87) (width 1.5) (layer "B.Cu") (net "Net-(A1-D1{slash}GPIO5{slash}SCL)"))
 (segment (start 88.313963 77.98) (end 94.69 77.98) (width 1.5) (layer "B.Cu") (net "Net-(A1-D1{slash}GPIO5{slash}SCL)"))
 (arc (start 71.04 96) (mid 71.22377 96.923879) (end 71.747106 97.707106) (width 1.5) (layer "B.Cu")
  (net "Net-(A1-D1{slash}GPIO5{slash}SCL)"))
 (arc (start 88.313963 77.98) (mid 86.231572 78.394213) (end 84.466207 79.573792) (width 1.5) (layer "B.Cu")
  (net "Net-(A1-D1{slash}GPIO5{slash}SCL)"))
 (arc (start 107.025 98.525) (mid 106.786855 98.684123) (end 106.505944 98.74) (width 1.5) (layer "B.Cu")
  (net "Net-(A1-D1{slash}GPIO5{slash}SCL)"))
 (arc (start 71.91 97.87) (mid 72.873655 98.513894) (end 74.010365 98.74) (width 1.5) (layer "B.Cu")
  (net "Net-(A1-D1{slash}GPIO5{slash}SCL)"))
 (arc (start 107.025 98.525) (mid 107.184123 98.286855) (end 107.24 98.005944) (width 1.5) (layer "B.Cu")
  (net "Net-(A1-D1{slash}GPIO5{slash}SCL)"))
 (arc (start 71.747106 92.292893) (mid 71.22377 93.07612) (end 71.04 94) (width 1.5) (layer "B.Cu")
  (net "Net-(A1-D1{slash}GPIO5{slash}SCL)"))
 (segment (start 88.903963 84.73) (end 95.901522 84.73) (width 1.5) (layer "B.Cu") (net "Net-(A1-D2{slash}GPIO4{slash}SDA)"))
 (segment (start 76.823502 93.1) (end 76.88 93.1) (width 1.5) (layer "B.Cu") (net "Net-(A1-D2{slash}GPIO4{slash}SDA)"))
 (segment (start 96.61 75.44) (end 94.69 75.44) (width 1.5) (layer "B.Cu") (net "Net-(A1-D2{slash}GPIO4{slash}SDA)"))
 (segment (start 81.825 95.105) (end 73.759246 95.105) (width 1.5) (layer "B.Cu") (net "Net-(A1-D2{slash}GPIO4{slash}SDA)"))
 (segment (start 100.34 81.776981) (end 100.34 81.423963) (width 1.5) (layer "B.Cu") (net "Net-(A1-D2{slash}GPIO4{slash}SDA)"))
 (segment (start 98.746195 77.576195) (end 96.61 75.44) (width 1.5) (layer "B.Cu") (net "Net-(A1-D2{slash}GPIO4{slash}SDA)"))
 (segment (start 73.6325 94.9475) (end 74.53 94.05) (width 1.5) (layer "B.Cu") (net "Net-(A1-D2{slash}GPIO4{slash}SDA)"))
 (segment (start 99.04 83.43) (end 100.090391 82.379608) (width 1.5) (layer "B.Cu") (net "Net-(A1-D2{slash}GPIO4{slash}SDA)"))
 (segment (start 79.269949 92.11005) (end 85.056207 86.323792) (width 1.5) (layer "B.Cu") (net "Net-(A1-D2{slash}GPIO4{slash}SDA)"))
 (arc (start 100.34 81.423963) (mid 99.925777 79.341558) (end 98.746195 77.576195) (width 1.5) (layer "B.Cu")
  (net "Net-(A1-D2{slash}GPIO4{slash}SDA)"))
 (arc (start 76.88 93.1) (mid 78.173431 92.84272) (end 79.269949 92.11005) (width 1.5) (layer "B.Cu")
  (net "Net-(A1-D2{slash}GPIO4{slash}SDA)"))
 (arc (start 73.6325 95.0525) (mid 73.610753 95) (end 73.6325 94.9475) (width 1.5) (layer "B.Cu") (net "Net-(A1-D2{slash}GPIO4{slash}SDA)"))
 (arc (start 85.056207 86.323792) (mid 86.821572 85.144213) (end 88.903963 84.73) (width 1.5) (layer "B.Cu")
  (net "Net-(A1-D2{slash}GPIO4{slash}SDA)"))
 (arc (start 73.759246 95.105) (mid 73.690651 95.091355) (end 73.6325 95.0525) (width 1.5) (layer "B.Cu")
  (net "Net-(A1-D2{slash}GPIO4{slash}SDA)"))
 (arc (start 95.901522 84.73) (mid 97.600064 84.392135) (end 99.04 83.43) (width 1.5) (layer "B.Cu")
  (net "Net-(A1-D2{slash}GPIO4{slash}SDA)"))
 (arc (start 74.53 94.05) (mid 75.582267 93.346896) (end 76.823502 93.1) (width 1.5) (layer "B.Cu")
  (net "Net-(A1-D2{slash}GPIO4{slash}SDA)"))
 (arc (start 100.090391 82.379608) (mid 100.275132 82.103119) (end 100.34 81.776981) (width 1.5) (layer "B.Cu")
  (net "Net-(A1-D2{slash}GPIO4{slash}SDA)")))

